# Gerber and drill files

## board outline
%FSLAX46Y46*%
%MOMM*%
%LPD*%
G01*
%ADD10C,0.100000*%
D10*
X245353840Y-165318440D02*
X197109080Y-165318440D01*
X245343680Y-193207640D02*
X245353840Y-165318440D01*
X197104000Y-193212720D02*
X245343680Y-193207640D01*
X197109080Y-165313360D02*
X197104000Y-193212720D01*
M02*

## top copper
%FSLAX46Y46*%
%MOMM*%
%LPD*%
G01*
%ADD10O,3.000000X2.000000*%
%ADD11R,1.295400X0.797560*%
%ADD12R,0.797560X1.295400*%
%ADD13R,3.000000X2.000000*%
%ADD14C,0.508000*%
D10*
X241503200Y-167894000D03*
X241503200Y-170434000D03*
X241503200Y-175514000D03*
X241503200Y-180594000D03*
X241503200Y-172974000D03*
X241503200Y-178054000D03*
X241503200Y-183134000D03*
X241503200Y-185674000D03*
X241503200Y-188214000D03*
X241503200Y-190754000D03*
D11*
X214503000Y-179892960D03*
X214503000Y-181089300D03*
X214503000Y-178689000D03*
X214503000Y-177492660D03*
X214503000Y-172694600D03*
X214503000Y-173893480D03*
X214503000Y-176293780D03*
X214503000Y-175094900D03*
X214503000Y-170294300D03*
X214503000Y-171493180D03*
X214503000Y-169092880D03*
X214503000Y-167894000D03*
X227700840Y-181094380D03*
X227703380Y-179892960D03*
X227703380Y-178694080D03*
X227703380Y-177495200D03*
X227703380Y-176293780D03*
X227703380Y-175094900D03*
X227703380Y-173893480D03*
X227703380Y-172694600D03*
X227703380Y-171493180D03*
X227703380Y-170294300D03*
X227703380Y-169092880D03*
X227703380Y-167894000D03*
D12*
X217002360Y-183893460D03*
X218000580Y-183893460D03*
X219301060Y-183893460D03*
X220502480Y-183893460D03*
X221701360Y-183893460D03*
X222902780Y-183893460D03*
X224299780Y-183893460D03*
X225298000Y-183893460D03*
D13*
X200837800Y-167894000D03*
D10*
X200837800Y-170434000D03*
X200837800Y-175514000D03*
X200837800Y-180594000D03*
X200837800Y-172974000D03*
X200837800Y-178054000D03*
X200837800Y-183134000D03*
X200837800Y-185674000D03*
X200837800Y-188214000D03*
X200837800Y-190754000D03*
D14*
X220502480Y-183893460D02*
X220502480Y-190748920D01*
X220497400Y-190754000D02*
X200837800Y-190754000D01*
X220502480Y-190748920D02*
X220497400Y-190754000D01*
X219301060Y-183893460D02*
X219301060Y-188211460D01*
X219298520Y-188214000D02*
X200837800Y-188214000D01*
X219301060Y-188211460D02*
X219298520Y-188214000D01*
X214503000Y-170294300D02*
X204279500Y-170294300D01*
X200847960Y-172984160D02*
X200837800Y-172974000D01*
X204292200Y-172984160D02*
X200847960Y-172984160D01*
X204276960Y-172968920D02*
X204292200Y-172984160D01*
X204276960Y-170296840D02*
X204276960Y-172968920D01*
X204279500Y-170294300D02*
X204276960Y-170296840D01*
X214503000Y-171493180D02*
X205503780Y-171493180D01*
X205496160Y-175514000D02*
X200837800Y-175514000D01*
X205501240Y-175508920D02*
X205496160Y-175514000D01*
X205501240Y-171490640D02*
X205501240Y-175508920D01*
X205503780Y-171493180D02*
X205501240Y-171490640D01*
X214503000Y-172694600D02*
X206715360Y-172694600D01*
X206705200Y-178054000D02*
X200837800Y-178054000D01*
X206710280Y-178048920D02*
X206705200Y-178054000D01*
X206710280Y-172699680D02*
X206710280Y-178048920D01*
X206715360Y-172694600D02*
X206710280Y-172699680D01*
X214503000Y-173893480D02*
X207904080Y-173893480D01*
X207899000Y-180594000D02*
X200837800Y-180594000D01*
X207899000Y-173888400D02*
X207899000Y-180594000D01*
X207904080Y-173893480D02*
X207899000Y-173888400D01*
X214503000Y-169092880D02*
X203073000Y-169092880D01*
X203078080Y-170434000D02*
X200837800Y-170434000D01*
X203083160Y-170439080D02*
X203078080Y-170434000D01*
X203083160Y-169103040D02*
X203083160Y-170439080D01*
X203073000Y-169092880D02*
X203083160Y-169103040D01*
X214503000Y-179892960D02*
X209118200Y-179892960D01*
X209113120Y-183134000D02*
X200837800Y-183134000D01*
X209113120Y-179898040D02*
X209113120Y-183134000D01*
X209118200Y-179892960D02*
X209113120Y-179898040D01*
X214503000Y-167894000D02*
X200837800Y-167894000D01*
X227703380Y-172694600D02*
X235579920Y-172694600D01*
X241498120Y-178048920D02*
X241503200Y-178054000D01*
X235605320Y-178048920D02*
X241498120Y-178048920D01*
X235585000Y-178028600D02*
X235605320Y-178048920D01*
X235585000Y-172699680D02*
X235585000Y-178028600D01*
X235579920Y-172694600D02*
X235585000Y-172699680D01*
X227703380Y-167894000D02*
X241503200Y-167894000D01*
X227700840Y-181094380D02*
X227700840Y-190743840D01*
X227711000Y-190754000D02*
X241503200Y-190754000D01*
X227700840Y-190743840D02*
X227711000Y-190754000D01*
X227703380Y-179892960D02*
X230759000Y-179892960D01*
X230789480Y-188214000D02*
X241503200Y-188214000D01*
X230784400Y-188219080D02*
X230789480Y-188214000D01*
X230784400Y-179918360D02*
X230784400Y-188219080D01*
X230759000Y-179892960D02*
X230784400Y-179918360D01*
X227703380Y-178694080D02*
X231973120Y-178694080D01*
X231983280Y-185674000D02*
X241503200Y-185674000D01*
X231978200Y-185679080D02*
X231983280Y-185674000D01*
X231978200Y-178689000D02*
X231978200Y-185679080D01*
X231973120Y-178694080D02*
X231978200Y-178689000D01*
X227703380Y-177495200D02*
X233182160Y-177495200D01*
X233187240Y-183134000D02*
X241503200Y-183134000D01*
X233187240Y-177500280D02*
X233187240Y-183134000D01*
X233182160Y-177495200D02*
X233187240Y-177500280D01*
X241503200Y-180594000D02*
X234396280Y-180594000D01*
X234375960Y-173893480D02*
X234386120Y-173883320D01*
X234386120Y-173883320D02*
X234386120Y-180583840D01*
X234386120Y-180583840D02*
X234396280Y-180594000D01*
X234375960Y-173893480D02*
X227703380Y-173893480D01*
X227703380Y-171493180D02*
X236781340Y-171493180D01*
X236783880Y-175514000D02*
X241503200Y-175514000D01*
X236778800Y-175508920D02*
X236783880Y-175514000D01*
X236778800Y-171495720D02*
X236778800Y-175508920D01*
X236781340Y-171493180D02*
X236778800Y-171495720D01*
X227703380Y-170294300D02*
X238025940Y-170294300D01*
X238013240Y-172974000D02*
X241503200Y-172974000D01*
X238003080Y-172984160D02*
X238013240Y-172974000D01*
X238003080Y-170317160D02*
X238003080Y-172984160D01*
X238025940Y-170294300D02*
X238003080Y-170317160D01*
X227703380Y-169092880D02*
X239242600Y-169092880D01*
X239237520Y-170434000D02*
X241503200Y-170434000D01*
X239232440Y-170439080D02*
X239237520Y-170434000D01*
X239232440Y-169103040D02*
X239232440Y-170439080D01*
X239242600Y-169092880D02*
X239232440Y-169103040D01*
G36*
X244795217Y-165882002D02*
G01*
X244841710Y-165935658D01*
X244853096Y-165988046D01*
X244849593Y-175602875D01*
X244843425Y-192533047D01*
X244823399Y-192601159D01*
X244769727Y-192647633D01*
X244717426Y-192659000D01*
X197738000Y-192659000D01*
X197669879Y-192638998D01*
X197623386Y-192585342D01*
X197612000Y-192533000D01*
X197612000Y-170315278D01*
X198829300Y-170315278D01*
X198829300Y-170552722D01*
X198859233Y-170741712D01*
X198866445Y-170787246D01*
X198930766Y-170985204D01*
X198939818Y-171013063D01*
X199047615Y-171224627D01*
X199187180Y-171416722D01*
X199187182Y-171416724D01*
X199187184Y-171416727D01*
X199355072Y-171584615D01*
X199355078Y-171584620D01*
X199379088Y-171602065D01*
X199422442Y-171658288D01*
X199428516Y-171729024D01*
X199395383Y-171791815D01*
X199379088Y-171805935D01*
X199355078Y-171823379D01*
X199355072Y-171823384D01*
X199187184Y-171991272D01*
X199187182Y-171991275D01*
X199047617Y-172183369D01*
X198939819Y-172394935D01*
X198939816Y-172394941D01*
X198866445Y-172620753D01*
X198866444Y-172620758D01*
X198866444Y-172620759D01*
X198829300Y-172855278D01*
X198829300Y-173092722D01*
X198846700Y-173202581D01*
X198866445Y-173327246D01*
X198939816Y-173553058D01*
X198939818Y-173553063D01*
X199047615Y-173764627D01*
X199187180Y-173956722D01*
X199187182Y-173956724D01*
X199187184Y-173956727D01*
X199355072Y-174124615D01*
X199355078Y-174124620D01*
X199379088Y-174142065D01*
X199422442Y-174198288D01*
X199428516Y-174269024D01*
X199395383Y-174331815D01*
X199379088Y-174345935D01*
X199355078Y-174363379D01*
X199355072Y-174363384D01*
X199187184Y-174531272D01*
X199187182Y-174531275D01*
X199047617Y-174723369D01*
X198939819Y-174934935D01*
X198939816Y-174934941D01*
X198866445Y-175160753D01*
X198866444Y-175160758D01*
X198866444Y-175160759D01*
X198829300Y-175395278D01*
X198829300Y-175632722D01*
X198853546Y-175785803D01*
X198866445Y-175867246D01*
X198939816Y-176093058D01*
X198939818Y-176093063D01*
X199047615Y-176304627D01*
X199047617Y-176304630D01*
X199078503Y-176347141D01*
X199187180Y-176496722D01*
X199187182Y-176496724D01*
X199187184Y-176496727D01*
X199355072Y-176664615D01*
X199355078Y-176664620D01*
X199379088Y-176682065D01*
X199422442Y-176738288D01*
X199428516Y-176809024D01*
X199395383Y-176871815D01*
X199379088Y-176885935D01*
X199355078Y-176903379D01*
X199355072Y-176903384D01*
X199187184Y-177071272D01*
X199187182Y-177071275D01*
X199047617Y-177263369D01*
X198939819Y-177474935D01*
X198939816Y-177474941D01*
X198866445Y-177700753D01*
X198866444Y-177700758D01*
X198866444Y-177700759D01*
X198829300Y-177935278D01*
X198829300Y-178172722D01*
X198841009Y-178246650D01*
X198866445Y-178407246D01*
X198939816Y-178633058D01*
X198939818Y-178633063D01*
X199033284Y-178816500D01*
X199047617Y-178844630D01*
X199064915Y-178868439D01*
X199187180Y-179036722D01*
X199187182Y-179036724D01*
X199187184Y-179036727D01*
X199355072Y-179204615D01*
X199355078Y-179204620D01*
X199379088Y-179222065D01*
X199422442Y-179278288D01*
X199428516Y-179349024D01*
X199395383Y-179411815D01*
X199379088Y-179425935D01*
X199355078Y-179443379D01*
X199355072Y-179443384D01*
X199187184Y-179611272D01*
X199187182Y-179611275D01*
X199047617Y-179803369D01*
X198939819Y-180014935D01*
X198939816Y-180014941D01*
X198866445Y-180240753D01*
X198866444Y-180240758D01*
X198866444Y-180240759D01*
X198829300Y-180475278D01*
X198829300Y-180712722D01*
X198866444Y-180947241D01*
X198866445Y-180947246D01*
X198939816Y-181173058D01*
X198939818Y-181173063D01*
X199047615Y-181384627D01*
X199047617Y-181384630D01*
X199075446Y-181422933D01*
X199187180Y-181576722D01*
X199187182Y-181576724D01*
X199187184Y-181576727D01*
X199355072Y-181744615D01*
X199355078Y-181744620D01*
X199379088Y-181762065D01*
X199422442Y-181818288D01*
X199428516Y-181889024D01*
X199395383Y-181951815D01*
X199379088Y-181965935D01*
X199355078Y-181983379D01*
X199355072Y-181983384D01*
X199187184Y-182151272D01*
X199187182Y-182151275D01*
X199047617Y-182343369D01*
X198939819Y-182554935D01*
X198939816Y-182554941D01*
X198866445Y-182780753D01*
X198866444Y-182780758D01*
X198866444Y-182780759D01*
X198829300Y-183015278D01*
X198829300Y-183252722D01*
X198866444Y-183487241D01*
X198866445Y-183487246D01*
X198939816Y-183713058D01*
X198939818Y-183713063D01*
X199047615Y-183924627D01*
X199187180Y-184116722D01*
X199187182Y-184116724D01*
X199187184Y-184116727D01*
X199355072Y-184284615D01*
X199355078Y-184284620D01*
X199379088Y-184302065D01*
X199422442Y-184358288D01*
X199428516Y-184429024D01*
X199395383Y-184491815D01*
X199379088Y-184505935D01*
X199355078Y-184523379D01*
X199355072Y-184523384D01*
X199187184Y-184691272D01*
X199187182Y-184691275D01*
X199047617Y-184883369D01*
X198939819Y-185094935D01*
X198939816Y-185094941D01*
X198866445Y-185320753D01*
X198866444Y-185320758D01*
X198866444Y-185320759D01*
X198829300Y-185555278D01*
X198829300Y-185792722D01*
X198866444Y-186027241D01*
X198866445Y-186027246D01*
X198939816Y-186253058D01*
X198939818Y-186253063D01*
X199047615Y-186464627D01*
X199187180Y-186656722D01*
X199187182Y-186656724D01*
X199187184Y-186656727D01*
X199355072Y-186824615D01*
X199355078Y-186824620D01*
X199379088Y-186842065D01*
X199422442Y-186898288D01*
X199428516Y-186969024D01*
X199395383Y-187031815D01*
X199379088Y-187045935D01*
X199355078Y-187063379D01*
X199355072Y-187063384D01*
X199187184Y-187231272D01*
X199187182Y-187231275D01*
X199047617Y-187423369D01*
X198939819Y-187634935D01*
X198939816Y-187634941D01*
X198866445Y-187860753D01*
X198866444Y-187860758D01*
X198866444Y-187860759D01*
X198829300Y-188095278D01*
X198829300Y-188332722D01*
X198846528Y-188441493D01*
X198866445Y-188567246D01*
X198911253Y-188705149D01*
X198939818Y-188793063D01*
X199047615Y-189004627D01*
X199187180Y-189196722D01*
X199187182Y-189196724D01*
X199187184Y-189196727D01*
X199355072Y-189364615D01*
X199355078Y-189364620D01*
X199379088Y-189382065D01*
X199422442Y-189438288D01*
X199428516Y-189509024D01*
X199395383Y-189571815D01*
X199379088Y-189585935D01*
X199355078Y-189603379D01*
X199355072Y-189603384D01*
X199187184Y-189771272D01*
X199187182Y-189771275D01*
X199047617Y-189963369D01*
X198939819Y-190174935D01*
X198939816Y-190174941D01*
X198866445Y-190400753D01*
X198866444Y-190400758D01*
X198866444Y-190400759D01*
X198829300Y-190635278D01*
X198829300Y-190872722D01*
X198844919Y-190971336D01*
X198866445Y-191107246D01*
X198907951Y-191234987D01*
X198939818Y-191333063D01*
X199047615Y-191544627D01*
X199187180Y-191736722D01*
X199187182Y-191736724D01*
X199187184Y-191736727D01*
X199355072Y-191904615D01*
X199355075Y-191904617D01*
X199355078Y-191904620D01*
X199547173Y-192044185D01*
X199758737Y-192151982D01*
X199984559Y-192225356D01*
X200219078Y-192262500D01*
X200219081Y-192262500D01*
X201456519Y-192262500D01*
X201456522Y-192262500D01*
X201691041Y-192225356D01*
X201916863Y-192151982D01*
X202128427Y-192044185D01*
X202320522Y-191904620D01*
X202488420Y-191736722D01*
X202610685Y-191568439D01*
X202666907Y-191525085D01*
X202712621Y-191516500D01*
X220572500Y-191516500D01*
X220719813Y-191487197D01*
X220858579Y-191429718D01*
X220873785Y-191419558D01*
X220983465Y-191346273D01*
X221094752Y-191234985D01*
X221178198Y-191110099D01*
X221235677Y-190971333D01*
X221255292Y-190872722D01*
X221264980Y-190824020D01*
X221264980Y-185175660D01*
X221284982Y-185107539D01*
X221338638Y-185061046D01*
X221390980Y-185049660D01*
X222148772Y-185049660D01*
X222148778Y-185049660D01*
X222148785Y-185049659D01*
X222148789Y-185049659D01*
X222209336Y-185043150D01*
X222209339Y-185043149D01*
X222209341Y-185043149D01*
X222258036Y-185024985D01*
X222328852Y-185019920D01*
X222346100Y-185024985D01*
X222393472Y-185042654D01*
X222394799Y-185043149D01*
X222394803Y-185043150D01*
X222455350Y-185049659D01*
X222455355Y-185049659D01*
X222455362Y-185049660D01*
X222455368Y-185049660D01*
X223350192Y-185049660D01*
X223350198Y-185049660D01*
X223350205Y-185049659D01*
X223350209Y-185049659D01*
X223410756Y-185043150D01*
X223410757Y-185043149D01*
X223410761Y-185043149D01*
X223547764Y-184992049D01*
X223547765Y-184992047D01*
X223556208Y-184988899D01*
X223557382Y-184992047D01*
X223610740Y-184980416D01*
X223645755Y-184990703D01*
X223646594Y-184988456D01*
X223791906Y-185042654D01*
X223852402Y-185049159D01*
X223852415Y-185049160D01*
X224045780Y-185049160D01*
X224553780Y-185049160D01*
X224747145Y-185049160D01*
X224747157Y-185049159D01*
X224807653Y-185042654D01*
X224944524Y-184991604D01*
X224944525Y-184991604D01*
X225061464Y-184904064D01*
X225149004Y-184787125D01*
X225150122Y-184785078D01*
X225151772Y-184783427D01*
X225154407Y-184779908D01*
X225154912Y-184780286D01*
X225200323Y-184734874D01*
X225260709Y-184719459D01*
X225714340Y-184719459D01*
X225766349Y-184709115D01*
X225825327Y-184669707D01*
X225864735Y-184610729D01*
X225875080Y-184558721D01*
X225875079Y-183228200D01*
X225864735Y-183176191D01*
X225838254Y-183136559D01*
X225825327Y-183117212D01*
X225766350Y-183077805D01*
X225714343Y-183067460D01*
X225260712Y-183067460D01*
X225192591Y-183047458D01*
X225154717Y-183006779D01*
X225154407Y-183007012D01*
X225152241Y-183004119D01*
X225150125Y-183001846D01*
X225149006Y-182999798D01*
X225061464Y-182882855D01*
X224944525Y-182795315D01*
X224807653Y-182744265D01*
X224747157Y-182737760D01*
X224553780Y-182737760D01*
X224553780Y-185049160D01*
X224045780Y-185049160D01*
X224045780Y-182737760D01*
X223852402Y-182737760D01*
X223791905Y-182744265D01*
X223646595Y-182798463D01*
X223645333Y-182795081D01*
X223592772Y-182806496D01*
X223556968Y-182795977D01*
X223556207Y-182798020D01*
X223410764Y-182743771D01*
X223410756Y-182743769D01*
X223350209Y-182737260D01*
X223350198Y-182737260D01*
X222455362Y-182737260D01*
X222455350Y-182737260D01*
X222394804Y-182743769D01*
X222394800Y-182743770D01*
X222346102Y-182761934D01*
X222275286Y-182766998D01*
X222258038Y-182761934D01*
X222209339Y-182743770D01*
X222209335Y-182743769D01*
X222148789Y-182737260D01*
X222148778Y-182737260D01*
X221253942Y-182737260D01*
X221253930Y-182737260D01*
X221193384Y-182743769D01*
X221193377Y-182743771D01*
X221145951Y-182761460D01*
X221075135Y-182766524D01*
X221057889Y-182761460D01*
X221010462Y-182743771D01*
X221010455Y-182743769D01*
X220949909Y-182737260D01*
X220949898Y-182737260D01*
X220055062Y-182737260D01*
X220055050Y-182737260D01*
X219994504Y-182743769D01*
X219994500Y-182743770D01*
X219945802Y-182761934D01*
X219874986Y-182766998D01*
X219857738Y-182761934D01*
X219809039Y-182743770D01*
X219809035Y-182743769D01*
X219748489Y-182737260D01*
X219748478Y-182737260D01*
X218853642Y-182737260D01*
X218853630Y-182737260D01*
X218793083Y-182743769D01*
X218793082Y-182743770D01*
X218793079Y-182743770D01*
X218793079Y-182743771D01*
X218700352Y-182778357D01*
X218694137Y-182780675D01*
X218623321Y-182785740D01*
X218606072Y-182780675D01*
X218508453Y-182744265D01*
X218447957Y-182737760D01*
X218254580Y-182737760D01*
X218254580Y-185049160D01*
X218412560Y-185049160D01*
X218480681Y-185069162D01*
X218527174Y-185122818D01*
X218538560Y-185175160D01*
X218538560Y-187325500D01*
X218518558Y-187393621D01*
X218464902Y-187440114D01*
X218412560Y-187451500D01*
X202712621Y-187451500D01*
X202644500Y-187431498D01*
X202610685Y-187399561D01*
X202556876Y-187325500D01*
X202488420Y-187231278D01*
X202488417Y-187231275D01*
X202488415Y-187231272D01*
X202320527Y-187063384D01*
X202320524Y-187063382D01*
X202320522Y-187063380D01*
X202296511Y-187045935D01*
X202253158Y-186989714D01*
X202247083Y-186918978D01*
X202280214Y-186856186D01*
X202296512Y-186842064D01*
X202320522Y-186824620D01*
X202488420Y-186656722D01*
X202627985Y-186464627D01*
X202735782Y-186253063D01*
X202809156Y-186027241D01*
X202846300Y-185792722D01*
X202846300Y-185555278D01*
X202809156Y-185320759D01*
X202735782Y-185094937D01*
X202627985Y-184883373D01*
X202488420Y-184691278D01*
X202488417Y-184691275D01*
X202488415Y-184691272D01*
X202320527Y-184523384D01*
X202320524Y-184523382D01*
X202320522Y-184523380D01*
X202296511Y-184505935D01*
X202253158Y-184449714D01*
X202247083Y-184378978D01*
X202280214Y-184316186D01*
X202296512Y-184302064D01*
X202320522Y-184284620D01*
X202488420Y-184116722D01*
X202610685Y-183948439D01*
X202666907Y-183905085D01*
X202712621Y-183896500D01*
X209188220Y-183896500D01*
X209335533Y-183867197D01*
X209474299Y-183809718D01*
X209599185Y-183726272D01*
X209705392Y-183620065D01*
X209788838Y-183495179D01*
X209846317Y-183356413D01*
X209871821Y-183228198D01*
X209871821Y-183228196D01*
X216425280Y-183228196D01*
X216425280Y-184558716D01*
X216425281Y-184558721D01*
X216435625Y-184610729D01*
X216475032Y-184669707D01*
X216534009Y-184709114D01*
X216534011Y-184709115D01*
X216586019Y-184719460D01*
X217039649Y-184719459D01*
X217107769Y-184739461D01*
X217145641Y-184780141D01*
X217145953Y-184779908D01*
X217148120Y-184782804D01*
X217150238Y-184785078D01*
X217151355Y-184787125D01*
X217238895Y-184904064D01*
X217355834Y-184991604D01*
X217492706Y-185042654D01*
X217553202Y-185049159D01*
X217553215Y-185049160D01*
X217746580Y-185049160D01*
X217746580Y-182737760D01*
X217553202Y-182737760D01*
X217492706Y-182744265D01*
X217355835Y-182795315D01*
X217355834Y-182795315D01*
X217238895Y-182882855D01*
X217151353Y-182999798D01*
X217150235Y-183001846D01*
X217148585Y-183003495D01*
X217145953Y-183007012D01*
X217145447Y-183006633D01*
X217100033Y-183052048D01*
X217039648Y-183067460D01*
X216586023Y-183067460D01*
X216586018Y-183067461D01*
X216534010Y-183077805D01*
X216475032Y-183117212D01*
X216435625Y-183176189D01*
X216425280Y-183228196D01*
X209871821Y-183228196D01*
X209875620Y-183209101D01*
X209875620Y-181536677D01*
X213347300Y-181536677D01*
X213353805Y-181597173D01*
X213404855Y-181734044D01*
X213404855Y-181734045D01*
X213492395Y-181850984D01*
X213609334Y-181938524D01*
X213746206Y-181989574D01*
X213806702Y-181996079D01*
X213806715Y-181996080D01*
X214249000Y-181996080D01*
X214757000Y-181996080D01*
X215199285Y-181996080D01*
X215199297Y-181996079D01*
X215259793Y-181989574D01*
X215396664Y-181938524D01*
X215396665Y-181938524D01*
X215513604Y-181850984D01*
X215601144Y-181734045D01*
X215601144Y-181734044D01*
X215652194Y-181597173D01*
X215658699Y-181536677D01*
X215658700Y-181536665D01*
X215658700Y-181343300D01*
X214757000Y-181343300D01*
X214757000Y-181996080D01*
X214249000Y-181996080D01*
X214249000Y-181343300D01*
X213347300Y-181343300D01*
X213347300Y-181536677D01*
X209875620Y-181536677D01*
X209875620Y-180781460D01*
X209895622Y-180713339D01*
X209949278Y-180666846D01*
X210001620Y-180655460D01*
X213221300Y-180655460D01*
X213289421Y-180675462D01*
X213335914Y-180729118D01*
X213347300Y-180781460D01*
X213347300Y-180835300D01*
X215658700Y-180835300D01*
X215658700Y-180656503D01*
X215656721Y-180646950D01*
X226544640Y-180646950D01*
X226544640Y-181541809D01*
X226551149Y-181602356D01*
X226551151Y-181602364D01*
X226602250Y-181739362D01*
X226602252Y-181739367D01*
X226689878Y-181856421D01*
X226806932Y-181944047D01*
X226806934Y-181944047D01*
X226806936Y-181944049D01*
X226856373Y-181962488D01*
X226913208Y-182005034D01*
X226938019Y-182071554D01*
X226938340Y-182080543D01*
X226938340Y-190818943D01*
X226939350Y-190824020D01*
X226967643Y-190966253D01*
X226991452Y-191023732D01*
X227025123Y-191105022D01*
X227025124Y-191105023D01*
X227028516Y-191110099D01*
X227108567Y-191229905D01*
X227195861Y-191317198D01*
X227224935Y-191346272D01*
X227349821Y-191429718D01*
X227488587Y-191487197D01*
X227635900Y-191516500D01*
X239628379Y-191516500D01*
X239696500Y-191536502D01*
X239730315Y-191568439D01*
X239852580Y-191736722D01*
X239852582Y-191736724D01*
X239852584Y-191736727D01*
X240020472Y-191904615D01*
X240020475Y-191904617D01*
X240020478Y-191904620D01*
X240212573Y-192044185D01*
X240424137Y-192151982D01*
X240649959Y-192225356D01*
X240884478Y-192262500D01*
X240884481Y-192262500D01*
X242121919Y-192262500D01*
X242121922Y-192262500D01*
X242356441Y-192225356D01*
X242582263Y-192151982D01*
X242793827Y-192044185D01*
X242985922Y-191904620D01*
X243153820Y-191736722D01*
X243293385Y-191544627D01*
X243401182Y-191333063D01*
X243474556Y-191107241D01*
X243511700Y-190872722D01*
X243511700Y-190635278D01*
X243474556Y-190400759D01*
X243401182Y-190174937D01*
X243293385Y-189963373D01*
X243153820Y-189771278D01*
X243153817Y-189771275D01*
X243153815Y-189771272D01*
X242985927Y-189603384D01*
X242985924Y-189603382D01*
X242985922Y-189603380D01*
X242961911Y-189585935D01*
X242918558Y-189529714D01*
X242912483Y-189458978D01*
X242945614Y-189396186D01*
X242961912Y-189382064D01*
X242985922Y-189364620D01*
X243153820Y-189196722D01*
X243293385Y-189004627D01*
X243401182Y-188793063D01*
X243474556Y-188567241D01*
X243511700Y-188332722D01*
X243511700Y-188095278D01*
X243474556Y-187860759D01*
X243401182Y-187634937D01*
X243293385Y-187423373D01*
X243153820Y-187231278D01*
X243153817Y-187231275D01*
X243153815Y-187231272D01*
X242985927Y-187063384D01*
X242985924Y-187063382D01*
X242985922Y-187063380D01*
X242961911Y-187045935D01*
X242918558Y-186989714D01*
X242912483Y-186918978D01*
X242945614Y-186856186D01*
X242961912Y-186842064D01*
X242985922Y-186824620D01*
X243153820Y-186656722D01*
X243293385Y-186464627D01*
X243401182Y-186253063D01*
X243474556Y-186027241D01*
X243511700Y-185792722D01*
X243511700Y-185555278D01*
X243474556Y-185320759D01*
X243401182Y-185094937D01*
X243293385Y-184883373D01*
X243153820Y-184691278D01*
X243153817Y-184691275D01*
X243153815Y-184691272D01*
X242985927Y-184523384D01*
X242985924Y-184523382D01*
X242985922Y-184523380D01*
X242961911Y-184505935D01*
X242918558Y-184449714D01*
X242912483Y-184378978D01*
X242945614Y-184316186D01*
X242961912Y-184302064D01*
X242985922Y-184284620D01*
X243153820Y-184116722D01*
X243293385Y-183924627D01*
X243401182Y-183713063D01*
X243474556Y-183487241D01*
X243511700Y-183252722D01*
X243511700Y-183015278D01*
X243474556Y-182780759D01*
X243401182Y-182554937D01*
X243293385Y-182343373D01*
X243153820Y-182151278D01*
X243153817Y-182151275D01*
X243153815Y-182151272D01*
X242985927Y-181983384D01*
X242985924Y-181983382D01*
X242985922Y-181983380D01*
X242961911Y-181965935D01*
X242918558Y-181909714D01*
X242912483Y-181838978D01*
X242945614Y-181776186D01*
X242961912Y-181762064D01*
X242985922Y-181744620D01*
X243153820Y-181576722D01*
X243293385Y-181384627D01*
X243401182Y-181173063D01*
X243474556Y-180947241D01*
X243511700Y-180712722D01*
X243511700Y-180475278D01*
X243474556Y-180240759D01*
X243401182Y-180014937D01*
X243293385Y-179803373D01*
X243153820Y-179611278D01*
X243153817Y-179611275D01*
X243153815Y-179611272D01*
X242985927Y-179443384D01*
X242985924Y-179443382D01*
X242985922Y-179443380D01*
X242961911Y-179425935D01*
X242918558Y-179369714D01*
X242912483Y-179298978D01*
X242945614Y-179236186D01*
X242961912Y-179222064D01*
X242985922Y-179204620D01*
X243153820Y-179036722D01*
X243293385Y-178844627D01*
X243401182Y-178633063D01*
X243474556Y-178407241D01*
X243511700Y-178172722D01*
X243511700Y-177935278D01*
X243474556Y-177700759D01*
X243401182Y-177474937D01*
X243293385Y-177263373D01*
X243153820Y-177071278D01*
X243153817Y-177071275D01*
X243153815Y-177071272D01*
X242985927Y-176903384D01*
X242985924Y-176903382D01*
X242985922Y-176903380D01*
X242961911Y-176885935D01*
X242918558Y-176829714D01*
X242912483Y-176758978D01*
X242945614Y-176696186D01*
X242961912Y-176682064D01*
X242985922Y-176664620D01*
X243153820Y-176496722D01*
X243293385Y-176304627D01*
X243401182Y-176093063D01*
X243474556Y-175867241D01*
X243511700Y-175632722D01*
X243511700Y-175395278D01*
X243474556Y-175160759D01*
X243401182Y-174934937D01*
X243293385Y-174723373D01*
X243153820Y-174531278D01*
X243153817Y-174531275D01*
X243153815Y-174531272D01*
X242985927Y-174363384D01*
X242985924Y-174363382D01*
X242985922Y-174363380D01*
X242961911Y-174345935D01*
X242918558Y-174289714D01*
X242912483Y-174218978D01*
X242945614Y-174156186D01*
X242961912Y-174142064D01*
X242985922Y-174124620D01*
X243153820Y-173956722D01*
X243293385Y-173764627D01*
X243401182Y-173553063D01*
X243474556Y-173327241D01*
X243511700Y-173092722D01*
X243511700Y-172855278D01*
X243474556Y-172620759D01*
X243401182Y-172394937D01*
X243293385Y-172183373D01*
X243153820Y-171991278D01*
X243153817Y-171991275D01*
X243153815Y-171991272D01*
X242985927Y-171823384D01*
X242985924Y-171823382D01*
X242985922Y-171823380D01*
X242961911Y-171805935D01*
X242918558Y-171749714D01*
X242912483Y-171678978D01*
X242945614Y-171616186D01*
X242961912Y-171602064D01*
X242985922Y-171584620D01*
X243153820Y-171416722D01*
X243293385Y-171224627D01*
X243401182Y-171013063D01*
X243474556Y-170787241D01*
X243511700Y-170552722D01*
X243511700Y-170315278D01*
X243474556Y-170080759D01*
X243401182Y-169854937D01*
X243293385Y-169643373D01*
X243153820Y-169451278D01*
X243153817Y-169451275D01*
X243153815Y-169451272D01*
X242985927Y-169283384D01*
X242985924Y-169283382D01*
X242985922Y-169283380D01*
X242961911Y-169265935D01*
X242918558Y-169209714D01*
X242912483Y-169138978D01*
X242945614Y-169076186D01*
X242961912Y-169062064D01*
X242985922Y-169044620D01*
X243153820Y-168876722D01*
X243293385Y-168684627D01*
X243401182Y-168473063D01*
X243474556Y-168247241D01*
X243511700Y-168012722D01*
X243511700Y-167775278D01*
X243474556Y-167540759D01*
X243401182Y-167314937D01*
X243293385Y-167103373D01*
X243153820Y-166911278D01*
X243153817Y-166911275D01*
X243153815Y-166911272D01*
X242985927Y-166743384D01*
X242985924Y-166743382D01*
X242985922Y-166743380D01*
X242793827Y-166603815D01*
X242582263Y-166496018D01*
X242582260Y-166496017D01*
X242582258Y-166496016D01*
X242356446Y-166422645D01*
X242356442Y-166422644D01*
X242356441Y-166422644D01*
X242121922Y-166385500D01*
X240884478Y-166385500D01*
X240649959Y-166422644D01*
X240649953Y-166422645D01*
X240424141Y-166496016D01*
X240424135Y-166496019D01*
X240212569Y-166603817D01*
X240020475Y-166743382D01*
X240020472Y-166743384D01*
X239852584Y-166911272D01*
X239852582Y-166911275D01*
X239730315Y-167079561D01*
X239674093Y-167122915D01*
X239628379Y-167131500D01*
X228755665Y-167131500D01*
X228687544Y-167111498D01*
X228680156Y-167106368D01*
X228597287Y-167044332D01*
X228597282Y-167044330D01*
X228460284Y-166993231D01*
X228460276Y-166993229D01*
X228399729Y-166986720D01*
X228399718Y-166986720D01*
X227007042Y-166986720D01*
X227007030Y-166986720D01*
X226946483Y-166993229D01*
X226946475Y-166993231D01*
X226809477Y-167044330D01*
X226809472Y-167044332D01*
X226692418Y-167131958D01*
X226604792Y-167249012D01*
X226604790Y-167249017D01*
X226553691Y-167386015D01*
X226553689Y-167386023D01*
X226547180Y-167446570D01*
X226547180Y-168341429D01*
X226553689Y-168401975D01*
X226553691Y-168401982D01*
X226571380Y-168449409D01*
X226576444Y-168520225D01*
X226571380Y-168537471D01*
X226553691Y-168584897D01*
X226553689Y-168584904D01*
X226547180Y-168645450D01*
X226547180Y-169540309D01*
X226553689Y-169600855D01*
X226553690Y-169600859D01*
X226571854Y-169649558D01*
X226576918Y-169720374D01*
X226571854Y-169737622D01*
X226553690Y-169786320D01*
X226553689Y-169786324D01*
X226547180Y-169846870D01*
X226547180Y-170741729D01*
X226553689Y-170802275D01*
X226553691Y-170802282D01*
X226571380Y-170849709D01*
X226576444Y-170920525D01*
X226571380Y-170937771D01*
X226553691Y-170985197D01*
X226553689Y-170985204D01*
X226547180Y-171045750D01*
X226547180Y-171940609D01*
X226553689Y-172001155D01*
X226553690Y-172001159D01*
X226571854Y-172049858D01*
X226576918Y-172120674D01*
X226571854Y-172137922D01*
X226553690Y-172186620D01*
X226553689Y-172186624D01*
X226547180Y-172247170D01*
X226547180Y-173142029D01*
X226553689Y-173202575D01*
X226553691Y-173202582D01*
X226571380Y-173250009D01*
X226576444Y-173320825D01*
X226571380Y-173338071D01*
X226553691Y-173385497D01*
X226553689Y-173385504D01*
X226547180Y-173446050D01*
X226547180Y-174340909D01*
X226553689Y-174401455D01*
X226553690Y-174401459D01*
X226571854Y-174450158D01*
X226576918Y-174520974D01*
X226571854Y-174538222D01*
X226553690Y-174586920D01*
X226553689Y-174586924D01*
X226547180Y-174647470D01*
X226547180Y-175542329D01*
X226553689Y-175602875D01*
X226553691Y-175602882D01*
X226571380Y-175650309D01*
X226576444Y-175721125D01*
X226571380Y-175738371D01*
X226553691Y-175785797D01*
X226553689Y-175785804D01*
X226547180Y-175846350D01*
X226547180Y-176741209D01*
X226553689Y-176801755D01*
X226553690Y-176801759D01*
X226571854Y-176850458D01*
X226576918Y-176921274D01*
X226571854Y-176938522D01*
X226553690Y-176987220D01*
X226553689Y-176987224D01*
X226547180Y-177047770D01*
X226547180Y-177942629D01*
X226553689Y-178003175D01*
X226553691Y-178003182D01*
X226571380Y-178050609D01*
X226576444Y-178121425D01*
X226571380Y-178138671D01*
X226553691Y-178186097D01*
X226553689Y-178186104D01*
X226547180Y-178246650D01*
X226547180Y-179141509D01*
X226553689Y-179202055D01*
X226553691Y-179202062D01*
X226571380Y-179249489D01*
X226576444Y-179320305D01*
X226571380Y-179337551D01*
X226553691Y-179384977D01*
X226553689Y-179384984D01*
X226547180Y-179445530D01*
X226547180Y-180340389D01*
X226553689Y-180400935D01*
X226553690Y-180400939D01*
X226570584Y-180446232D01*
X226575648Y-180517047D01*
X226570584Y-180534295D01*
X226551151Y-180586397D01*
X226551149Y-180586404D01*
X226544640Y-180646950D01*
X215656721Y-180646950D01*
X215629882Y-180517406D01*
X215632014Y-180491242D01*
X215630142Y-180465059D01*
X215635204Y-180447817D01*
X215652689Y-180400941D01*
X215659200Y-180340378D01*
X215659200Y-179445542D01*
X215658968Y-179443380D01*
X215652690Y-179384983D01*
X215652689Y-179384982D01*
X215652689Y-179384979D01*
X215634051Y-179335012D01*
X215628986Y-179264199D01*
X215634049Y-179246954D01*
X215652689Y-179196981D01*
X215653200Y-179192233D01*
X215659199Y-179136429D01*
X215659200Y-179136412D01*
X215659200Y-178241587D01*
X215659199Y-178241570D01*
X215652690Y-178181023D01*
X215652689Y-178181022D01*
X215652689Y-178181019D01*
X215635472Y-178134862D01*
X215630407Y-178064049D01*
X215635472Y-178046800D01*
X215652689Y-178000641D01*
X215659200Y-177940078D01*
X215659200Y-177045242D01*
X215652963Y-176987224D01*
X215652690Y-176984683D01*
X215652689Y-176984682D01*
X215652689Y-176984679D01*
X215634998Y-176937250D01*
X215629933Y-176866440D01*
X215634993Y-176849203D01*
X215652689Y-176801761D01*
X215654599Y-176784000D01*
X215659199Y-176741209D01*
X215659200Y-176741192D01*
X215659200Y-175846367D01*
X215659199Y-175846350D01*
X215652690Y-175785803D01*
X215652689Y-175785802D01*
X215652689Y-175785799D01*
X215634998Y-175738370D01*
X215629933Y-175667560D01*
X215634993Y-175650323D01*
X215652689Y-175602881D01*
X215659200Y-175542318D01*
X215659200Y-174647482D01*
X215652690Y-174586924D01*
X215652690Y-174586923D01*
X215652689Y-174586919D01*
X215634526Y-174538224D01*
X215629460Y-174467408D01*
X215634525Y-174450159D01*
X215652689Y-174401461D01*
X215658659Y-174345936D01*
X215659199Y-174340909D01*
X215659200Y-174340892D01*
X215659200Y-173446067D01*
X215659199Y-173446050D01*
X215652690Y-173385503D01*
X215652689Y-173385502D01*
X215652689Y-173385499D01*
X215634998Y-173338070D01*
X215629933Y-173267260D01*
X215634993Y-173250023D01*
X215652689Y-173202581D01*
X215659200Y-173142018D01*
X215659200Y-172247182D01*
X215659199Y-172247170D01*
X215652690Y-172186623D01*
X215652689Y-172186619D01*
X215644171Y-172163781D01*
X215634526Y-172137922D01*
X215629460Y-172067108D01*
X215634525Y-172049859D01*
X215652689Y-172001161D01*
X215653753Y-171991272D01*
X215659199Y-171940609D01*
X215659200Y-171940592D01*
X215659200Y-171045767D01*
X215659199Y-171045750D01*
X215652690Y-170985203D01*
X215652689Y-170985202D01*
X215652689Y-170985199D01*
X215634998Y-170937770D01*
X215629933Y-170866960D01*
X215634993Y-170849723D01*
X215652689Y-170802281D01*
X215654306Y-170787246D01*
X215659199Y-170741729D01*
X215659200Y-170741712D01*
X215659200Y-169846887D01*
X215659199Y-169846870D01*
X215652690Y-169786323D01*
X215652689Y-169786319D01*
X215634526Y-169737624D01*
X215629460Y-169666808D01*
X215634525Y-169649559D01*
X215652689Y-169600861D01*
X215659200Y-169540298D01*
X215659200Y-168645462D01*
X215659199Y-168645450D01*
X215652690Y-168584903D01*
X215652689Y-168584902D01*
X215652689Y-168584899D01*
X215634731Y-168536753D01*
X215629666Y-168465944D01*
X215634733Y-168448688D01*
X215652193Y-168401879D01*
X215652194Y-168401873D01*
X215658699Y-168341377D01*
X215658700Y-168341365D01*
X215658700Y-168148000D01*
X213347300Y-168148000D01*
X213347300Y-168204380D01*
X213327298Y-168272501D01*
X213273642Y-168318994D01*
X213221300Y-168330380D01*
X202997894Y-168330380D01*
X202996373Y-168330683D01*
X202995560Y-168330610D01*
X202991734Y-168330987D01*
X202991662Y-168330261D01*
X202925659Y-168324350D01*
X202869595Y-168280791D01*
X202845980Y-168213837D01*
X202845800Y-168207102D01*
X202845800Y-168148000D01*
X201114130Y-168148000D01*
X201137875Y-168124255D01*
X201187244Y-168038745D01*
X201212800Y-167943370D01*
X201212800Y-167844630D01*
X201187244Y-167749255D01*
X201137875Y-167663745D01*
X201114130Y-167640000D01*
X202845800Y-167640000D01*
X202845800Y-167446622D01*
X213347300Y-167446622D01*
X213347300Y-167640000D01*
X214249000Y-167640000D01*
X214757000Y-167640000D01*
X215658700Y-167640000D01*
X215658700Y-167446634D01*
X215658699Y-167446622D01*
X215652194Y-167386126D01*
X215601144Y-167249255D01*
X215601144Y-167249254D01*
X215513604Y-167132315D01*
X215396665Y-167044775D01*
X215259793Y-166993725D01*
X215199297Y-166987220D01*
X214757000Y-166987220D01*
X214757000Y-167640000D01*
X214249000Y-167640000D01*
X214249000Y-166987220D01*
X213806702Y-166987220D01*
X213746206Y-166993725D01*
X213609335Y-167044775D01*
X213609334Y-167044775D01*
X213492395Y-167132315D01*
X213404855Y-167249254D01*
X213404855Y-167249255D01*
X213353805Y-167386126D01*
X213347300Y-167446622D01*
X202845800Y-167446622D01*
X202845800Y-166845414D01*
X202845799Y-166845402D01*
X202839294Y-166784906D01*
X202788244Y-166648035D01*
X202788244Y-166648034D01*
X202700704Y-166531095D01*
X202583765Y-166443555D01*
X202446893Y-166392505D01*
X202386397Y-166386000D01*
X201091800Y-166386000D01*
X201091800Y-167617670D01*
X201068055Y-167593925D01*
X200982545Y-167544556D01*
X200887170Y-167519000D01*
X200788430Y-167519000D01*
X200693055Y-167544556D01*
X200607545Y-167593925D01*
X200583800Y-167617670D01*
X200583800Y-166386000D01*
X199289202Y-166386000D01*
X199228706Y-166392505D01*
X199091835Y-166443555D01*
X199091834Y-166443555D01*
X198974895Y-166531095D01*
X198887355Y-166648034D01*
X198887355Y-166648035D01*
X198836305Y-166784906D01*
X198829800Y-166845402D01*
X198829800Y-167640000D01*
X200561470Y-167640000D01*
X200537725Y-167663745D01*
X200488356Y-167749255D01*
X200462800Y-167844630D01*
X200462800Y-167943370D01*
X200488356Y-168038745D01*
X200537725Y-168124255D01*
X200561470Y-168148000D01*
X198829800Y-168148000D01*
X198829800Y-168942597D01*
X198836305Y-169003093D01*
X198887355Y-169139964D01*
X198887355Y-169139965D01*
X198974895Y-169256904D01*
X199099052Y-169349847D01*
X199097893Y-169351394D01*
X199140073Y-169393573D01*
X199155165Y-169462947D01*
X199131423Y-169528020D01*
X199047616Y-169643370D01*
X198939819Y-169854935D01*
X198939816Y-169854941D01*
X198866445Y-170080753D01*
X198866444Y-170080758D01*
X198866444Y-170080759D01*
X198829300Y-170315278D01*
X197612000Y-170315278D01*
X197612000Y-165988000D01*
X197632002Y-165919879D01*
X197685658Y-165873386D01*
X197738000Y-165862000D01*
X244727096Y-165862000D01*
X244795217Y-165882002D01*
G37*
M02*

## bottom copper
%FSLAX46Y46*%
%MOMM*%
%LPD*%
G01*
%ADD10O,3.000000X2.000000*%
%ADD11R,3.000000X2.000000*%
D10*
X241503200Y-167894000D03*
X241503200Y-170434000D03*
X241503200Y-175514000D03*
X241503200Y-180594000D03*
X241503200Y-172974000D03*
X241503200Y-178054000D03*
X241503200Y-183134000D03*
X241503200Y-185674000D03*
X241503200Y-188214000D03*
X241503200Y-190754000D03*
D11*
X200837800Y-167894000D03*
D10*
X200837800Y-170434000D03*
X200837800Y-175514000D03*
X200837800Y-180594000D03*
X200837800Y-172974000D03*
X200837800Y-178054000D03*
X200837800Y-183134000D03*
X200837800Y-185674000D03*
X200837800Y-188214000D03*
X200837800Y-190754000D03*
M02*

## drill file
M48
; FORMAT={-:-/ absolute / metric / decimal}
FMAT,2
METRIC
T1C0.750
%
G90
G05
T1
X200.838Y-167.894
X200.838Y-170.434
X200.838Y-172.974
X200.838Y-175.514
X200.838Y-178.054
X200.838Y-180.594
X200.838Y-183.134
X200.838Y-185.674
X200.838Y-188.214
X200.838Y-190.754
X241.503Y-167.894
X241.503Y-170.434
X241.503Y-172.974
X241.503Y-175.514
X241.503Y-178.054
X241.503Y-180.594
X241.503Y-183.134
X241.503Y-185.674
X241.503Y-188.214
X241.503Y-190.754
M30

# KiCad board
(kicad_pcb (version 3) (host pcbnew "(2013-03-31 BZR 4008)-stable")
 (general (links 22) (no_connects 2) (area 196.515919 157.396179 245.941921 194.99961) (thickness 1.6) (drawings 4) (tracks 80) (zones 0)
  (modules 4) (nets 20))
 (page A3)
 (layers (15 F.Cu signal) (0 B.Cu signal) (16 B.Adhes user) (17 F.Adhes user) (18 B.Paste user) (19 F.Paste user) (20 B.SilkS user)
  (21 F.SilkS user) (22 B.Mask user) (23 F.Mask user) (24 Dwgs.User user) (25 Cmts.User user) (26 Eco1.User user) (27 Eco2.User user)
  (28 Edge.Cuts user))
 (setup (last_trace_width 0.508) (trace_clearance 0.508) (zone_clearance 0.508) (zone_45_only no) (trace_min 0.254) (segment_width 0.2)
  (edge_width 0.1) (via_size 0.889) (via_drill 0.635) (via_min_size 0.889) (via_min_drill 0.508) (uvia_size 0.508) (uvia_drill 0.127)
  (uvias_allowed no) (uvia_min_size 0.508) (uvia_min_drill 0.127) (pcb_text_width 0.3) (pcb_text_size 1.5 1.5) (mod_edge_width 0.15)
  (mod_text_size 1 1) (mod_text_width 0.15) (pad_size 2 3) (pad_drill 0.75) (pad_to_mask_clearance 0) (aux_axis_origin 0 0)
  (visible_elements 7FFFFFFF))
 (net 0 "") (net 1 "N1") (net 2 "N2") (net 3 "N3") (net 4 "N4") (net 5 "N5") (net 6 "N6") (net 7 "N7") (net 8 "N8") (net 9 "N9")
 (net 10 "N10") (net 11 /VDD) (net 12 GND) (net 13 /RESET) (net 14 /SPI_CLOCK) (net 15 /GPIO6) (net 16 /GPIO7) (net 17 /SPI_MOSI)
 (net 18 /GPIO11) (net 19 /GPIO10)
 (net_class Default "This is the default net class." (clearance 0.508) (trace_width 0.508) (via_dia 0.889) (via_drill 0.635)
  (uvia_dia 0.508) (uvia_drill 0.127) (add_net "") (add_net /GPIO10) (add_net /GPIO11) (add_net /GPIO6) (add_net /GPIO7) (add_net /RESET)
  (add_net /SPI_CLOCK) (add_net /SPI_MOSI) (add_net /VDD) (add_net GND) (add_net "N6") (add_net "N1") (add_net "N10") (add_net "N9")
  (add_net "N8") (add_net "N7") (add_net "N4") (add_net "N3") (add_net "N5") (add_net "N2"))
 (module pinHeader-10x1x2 (layer F.Cu) (at 241.5032 179.324 270)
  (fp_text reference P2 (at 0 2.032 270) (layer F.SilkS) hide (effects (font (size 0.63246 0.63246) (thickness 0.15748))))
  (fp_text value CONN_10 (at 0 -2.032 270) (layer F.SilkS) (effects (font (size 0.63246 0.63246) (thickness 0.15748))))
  (pad 1 thru_hole oval (at -11.43 0 270) (size 2 3) (drill 0.75) (layers *.Cu *.Mask F.SilkS) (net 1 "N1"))
  (pad 2 thru_hole oval (at -8.89 0 270) (size 2 3) (drill 0.75) (layers *.Cu *.Mask F.SilkS) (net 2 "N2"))
  (pad 4 thru_hole oval (at -3.81 0 270) (size 2 3) (drill 0.75) (layers *.Cu *.Mask F.SilkS) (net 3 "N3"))
  (pad 6 thru_hole oval (at 1.27 0 270) (size 2 3) (drill 0.75) (layers *.Cu *.Mask F.SilkS) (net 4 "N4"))
  (pad 3 thru_hole oval (at -6.35 0 270) (size 2 3) (drill 0.75) (layers *.Cu *.Mask F.SilkS) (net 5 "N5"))
  (pad 5 thru_hole oval (at -1.27 0 270) (size 2 3) (drill 0.75) (layers *.Cu *.Mask F.SilkS) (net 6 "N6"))
  (pad 7 thru_hole oval (at 3.81 0 270) (size 2 3) (drill 0.75) (layers *.Cu *.Mask F.SilkS) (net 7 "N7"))
  (pad 8 thru_hole oval (at 6.35 0 270) (size 2 3) (drill 0.75) (layers *.Cu *.Mask F.SilkS) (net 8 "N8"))
  (pad 9 thru_hole oval (at 8.89 0 270) (size 2 3) (drill 0.75) (layers *.Cu *.Mask F.SilkS) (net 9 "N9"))
  (pad 10 thru_hole oval (at 11.43 0 270) (size 2 3) (drill 0.75) (layers *.Cu *.Mask F.SilkS) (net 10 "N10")))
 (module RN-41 (layer F.Cu) (at 214.503 167.894)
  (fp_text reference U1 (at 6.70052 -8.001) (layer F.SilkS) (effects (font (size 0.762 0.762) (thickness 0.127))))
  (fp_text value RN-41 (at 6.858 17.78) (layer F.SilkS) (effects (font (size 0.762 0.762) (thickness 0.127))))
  (pad 11 smd rect (at 0 11.99896) (size 1.2954 0.79756) (layers F.Cu F.Paste F.Mask) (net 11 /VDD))
  (pad 12 smd rect (at 0 13.1953) (size 1.2954 0.79756) (layers F.Cu F.Paste F.Mask) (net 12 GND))
  (pad 10 smd rect (at 0 10.795) (size 1.2954 0.79756) (layers F.Cu F.Paste F.Mask))
  (pad 9 smd rect (at 0 9.59866) (size 1.2954 0.79756) (layers F.Cu F.Paste F.Mask))
  (pad 5 smd rect (at 0 4.8006) (size 1.2954 0.79756) (layers F.Cu F.Paste F.Mask) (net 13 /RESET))
  (pad 6 smd rect (at 0 5.99948) (size 1.2954 0.79756) (layers F.Cu F.Paste F.Mask) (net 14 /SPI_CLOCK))
  (pad 8 smd rect (at 0 8.39978) (size 1.2954 0.79756) (layers F.Cu F.Paste F.Mask))
  (pad 7 smd rect (at 0 7.2009) (size 1.2954 0.79756) (layers F.Cu F.Paste F.Mask))
  (pad 3 smd rect (at 0 2.4003) (size 1.2954 0.79756) (layers F.Cu F.Paste F.Mask) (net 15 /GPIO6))
  (pad 4 smd rect (at 0 3.59918) (size 1.2954 0.79756) (layers F.Cu F.Paste F.Mask) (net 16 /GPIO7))
  (pad 2 smd rect (at 0 1.19888) (size 1.2954 0.79756) (layers F.Cu F.Paste F.Mask) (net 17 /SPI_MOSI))
  (pad 1 smd rect (at 0 0) (size 1.2954 0.79756) (layers F.Cu F.Paste F.Mask) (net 12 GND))
  (pad 13 smd rect (at 13.19784 13.20038) (size 1.2954 0.79756) (layers F.Cu F.Paste F.Mask) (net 10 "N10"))
  (pad 14 smd rect (at 13.20038 11.99896) (size 1.2954 0.79756) (layers F.Cu F.Paste F.Mask) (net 9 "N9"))
  (pad 15 smd rect (at 13.20038 10.80008) (size 1.2954 0.79756) (layers F.Cu F.Paste F.Mask) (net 8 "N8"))
  (pad 16 smd rect (at 13.20038 9.6012) (size 1.2954 0.79756) (layers F.Cu F.Paste F.Mask) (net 7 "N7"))
  (pad 17 smd rect (at 13.20038 8.39978) (size 1.2954 0.79756) (layers F.Cu F.Paste F.Mask))
  (pad 18 smd rect (at 13.20038 7.2009) (size 1.2954 0.79756) (layers F.Cu F.Paste F.Mask))
  (pad 19 smd rect (at 13.20038 5.99948) (size 1.2954 0.79756) (layers F.Cu F.Paste F.Mask) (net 4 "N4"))
  (pad 20 smd rect (at 13.20038 4.8006) (size 1.2954 0.79756) (layers F.Cu F.Paste F.Mask) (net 6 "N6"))
  (pad 21 smd rect (at 13.20038 3.59918) (size 1.2954 0.79756) (layers F.Cu F.Paste F.Mask) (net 3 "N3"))
  (pad 22 smd rect (at 13.20038 2.4003) (size 1.2954 0.79756) (layers F.Cu F.Paste F.Mask) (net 5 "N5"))
  (pad 23 smd rect (at 13.20038 1.19888) (size 1.2954 0.79756) (layers F.Cu F.Paste F.Mask) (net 2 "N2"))
  (pad 24 smd rect (at 13.20038 0) (size 1.2954 0.79756) (layers F.Cu F.Paste F.Mask) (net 1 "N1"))
  (pad 35 smd rect (at 2.49936 15.99946) (size 0.79756 1.2954) (layers F.Cu F.Paste F.Mask) (clearance 0.1778))
  (pad 29 smd rect (at 3.49758 15.99946) (size 0.79756 1.2954) (layers F.Cu F.Paste F.Mask) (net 12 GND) (clearance 0.1778))
  (pad 34 smd rect (at 4.79806 15.99946) (size 0.79756 1.2954) (layers F.Cu F.Paste F.Mask) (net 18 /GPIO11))
  (pad 33 smd rect (at 5.99948 15.99946) (size 0.79756 1.2954) (layers F.Cu F.Paste F.Mask) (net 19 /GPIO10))
  (pad 32 smd rect (at 7.19836 15.99946) (size 0.79756 1.2954) (layers F.Cu F.Paste F.Mask))
  (pad 31 smd rect (at 8.39978 15.99946) (size 0.79756 1.2954) (layers F.Cu F.Paste F.Mask))
  (pad 28 smd rect (at 9.79678 15.99946) (size 0.79756 1.2954) (layers F.Cu F.Paste F.Mask) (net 12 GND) (clearance 0.1778))
  (pad 30 smd rect (at 10.795 15.99946) (size 0.79756 1.2954) (layers F.Cu F.Paste F.Mask) (clearance 0.1778)))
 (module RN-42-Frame (layer F.Cu) (at 221.22892 179.26304)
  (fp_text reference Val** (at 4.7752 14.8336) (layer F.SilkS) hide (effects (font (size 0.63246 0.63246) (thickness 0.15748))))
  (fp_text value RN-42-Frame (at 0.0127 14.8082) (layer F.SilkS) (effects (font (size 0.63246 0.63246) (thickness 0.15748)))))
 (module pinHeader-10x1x (layer F.Cu) (at 200.8378 179.324 270)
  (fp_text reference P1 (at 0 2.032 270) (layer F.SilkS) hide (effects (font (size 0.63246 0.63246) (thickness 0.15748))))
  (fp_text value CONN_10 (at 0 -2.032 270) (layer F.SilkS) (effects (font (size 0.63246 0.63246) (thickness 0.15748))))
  (pad 1 thru_hole rect (at -11.43 0 270) (size 2 3) (drill 0.75) (layers *.Cu *.Mask F.SilkS) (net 12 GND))
  (pad 2 thru_hole oval (at -8.89 0 270) (size 2 3) (drill 0.75) (layers *.Cu *.Mask F.SilkS) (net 17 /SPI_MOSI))
  (pad 4 thru_hole oval (at -3.81 0 270) (size 2 3) (drill 0.75) (layers *.Cu *.Mask F.SilkS) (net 16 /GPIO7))
  (pad 6 thru_hole oval (at 1.27 0 270) (size 2 3) (drill 0.75) (layers *.Cu *.Mask F.SilkS) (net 14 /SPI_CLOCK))
  (pad 3 thru_hole oval (at -6.35 0 270) (size 2 3) (drill 0.75) (layers *.Cu *.Mask F.SilkS) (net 15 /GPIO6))
  (pad 5 thru_hole oval (at -1.27 0 270) (size 2 3) (drill 0.75) (layers *.Cu *.Mask F.SilkS) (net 13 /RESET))
  (pad 7 thru_hole oval (at 3.81 0 270) (size 2 3) (drill 0.75) (layers *.Cu *.Mask F.SilkS) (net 11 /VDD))
  (pad 8 thru_hole oval (at 6.35 0 270) (size 2 3) (drill 0.75) (layers *.Cu *.Mask F.SilkS))
  (pad 9 thru_hole oval (at 8.89 0 270) (size 2 3) (drill 0.75) (layers *.Cu *.Mask F.SilkS) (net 18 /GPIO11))
  (pad 10 thru_hole oval (at 11.43 0 270) (size 2 3) (drill 0.75) (layers *.Cu *.Mask F.SilkS) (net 19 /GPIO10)))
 (gr_line (start 245.35384 165.31844) (end 197.10908 165.31844) (angle 90) (layer Edge.Cuts) (width 0.1))
 (gr_line (start 245.34368 193.20764) (end 245.35384 165.31844) (angle 90) (layer Edge.Cuts) (width 0.1))
 (gr_line (start 197.104 193.21272) (end 245.34368 193.20764) (angle 90) (layer Edge.Cuts) (width 0.1))
 (gr_line (start 197.10908 165.31336) (end 197.104 193.21272) (angle 90) (layer Edge.Cuts) (width 0.1))
 (segment (start 220.50248 183.89346) (end 220.50248 190.74892) (width 0.508) (layer F.Cu) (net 19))
 (segment (start 220.4974 190.754) (end 200.8378 190.754) (width 0.508) (layer F.Cu) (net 19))
 (segment (start 220.50248 190.74892) (end 220.4974 190.754) (width 0.508) (layer F.Cu) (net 19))
 (segment (start 219.30106 183.89346) (end 219.30106 188.21146) (width 0.508) (layer F.Cu) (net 18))
 (segment (start 219.29852 188.214) (end 200.8378 188.214) (width 0.508) (layer F.Cu) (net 18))
 (segment (start 219.30106 188.21146) (end 219.29852 188.214) (width 0.508) (layer F.Cu) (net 18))
 (segment (start 214.503 170.2943) (end 204.2795 170.2943) (width 0.508) (layer F.Cu) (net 15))
 (segment (start 200.84796 172.98416) (end 200.8378 172.974) (width 0.508) (layer F.Cu) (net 15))
 (segment (start 204.2922 172.98416) (end 200.84796 172.98416) (width 0.508) (layer F.Cu) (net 15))
 (segment (start 204.27696 172.96892) (end 204.2922 172.98416) (width 0.508) (layer F.Cu) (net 15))
 (segment (start 204.27696 170.29684) (end 204.27696 172.96892) (width 0.508) (layer F.Cu) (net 15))
 (segment (start 204.2795 170.2943) (end 204.27696 170.29684) (width 0.508) (layer F.Cu) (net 15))
 (segment (start 214.503 171.49318) (end 205.50378 171.49318) (width 0.508) (layer F.Cu) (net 16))
 (segment (start 205.49616 175.514) (end 200.8378 175.514) (width 0.508) (layer F.Cu) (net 16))
 (segment (start 205.50124 175.50892) (end 205.49616 175.514) (width 0.508) (layer F.Cu) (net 16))
 (segment (start 205.50124 171.49064) (end 205.50124 175.50892) (width 0.508) (layer F.Cu) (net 16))
 (segment (start 205.50378 171.49318) (end 205.50124 171.49064) (width 0.508) (layer F.Cu) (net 16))
 (segment (start 214.503 172.6946) (end 206.71536 172.6946) (width 0.508) (layer F.Cu) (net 13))
 (segment (start 206.7052 178.054) (end 200.8378 178.054) (width 0.508) (layer F.Cu) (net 13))
 (segment (start 206.71028 178.04892) (end 206.7052 178.054) (width 0.508) (layer F.Cu) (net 13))
 (segment (start 206.71028 172.69968) (end 206.71028 178.04892) (width 0.508) (layer F.Cu) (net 13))
 (segment (start 206.71536 172.6946) (end 206.71028 172.69968) (width 0.508) (layer F.Cu) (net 13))
 (segment (start 214.503 173.89348) (end 207.90408 173.89348) (width 0.508) (layer F.Cu) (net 14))
 (segment (start 207.899 180.594) (end 200.8378 180.594) (width 0.508) (layer F.Cu) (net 14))
 (segment (start 207.899 173.8884) (end 207.899 180.594) (width 0.508) (layer F.Cu) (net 14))
 (segment (start 207.90408 173.89348) (end 207.899 173.8884) (width 0.508) (layer F.Cu) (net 14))
 (segment (start 214.503 169.09288) (end 203.073 169.09288) (width 0.508) (layer F.Cu) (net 17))
 (segment (start 203.07808 170.434) (end 200.8378 170.434) (width 0.508) (layer F.Cu) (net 17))
 (segment (start 203.08316 170.43908) (end 203.07808 170.434) (width 0.508) (layer F.Cu) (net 17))
 (segment (start 203.08316 169.10304) (end 203.08316 170.43908) (width 0.508) (layer F.Cu) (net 17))
 (segment (start 203.073 169.09288) (end 203.08316 169.10304) (width 0.508) (layer F.Cu) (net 17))
 (segment (start 214.503 179.89296) (end 209.1182 179.89296) (width 0.508) (layer F.Cu) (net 11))
 (segment (start 209.11312 183.134) (end 200.8378 183.134) (width 0.508) (layer F.Cu) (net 11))
 (segment (start 209.11312 179.89804) (end 209.11312 183.134) (width 0.508) (layer F.Cu) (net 11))
 (segment (start 209.1182 179.89296) (end 209.11312 179.89804) (width 0.508) (layer F.Cu) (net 11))
 (segment (start 214.503 167.894) (end 200.8378 167.894) (width 0.508) (layer F.Cu) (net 12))
 (segment (start 227.70338 172.6946) (end 235.57992 172.6946) (width 0.508) (layer F.Cu) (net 6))
 (segment (start 241.49812 178.04892) (end 241.5032 178.054) (width 0.508) (layer F.Cu) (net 6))
 (segment (start 235.60532 178.04892) (end 241.49812 178.04892) (width 0.508) (layer F.Cu) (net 6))
 (segment (start 235.585 178.0286) (end 235.60532 178.04892) (width 0.508) (layer F.Cu) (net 6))
 (segment (start 235.585 172.69968) (end 235.585 178.0286) (width 0.508) (layer F.Cu) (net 6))
 (segment (start 235.57992 172.6946) (end 235.585 172.69968) (width 0.508) (layer F.Cu) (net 6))
 (segment (start 227.70338 167.894) (end 241.5032 167.894) (width 0.508) (layer F.Cu) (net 1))
 (segment (start 227.70084 181.09438) (end 227.70084 190.74384) (width 0.508) (layer F.Cu) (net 10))
 (segment (start 227.711 190.754) (end 241.5032 190.754) (width 0.508) (layer F.Cu) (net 10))
 (segment (start 227.70084 190.74384) (end 227.711 190.754) (width 0.508) (layer F.Cu) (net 10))
 (segment (start 227.70338 179.89296) (end 230.759 179.89296) (width 0.508) (layer F.Cu) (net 9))
 (segment (start 230.78948 188.214) (end 241.5032 188.214) (width 0.508) (layer F.Cu) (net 9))
 (segment (start 230.7844 188.21908) (end 230.78948 188.214) (width 0.508) (layer F.Cu) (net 9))
 (segment (start 230.7844 179.91836) (end 230.7844 188.21908) (width 0.508) (layer F.Cu) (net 9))
 (segment (start 230.759 179.89296) (end 230.7844 179.91836) (width 0.508) (layer F.Cu) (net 9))
 (segment (start 227.70338 178.69408) (end 231.97312 178.69408) (width 0.508) (layer F.Cu) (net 8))
 (segment (start 231.98328 185.674) (end 241.5032 185.674) (width 0.508) (layer F.Cu) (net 8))
 (segment (start 231.9782 185.67908) (end 231.98328 185.674) (width 0.508) (layer F.Cu) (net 8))
 (segment (start 231.9782 178.689) (end 231.9782 185.67908) (width 0.508) (layer F.Cu) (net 8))
 (segment (start 231.97312 178.69408) (end 231.9782 178.689) (width 0.508) (layer F.Cu) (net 8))
 (segment (start 227.70338 177.4952) (end 233.18216 177.4952) (width 0.508) (layer F.Cu) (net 7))
 (segment (start 233.18724 183.134) (end 241.5032 183.134) (width 0.508) (layer F.Cu) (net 7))
 (segment (start 233.18724 177.50028) (end 233.18724 183.134) (width 0.508) (layer F.Cu) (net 7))
 (segment (start 233.18216 177.4952) (end 233.18724 177.50028) (width 0.508) (layer F.Cu) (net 7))
 (segment (start 241.5032 180.594) (end 234.39628 180.594) (width 0.508) (layer F.Cu) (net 4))
 (segment (start 234.37596 173.89348) (end 234.38612 173.88332) (width 0.508) (layer F.Cu) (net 4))
 (segment (start 234.38612 173.88332) (end 234.38612 180.58384) (width 0.508) (layer F.Cu) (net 4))
 (segment (start 234.38612 180.58384) (end 234.39628 180.594) (width 0.508) (layer F.Cu) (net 4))
 (segment (start 234.37596 173.89348) (end 227.70338 173.89348) (width 0.508) (layer F.Cu) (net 4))
 (segment (start 227.70338 171.49318) (end 236.78134 171.49318) (width 0.508) (layer F.Cu) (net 3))
 (segment (start 236.78388 175.514) (end 241.5032 175.514) (width 0.508) (layer F.Cu) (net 3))
 (segment (start 236.7788 175.50892) (end 236.78388 175.514) (width 0.508) (layer F.Cu) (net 3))
 (segment (start 236.7788 171.49572) (end 236.7788 175.50892) (width 0.508) (layer F.Cu) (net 3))
 (segment (start 236.78134 171.49318) (end 236.7788 171.49572) (width 0.508) (layer F.Cu) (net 3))
 (segment (start 227.70338 170.2943) (end 238.02594 170.2943) (width 0.508) (layer F.Cu) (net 5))
 (segment (start 238.01324 172.974) (end 241.5032 172.974) (width 0.508) (layer F.Cu) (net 5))
 (segment (start 238.00308 172.98416) (end 238.01324 172.974) (width 0.508) (layer F.Cu) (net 5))
 (segment (start 238.00308 170.31716) (end 238.00308 172.98416) (width 0.508) (layer F.Cu) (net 5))
 (segment (start 238.02594 170.2943) (end 238.00308 170.31716) (width 0.508) (layer F.Cu) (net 5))
 (segment (start 227.70338 169.09288) (end 239.2426 169.09288) (width 0.508) (layer F.Cu) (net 2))
 (segment (start 239.23752 170.434) (end 241.5032 170.434) (width 0.508) (layer F.Cu) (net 2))
 (segment (start 239.23244 170.43908) (end 239.23752 170.434) (width 0.508) (layer F.Cu) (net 2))
 (segment (start 239.23244 169.10304) (end 239.23244 170.43908) (width 0.508) (layer F.Cu) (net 2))
 (segment (start 239.2426 169.09288) (end 239.23244 169.10304) (width 0.508) (layer F.Cu) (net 2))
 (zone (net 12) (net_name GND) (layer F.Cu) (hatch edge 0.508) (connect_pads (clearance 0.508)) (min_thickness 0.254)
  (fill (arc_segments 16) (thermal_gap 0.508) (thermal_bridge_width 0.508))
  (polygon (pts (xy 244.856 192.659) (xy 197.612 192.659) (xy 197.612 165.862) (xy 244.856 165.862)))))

